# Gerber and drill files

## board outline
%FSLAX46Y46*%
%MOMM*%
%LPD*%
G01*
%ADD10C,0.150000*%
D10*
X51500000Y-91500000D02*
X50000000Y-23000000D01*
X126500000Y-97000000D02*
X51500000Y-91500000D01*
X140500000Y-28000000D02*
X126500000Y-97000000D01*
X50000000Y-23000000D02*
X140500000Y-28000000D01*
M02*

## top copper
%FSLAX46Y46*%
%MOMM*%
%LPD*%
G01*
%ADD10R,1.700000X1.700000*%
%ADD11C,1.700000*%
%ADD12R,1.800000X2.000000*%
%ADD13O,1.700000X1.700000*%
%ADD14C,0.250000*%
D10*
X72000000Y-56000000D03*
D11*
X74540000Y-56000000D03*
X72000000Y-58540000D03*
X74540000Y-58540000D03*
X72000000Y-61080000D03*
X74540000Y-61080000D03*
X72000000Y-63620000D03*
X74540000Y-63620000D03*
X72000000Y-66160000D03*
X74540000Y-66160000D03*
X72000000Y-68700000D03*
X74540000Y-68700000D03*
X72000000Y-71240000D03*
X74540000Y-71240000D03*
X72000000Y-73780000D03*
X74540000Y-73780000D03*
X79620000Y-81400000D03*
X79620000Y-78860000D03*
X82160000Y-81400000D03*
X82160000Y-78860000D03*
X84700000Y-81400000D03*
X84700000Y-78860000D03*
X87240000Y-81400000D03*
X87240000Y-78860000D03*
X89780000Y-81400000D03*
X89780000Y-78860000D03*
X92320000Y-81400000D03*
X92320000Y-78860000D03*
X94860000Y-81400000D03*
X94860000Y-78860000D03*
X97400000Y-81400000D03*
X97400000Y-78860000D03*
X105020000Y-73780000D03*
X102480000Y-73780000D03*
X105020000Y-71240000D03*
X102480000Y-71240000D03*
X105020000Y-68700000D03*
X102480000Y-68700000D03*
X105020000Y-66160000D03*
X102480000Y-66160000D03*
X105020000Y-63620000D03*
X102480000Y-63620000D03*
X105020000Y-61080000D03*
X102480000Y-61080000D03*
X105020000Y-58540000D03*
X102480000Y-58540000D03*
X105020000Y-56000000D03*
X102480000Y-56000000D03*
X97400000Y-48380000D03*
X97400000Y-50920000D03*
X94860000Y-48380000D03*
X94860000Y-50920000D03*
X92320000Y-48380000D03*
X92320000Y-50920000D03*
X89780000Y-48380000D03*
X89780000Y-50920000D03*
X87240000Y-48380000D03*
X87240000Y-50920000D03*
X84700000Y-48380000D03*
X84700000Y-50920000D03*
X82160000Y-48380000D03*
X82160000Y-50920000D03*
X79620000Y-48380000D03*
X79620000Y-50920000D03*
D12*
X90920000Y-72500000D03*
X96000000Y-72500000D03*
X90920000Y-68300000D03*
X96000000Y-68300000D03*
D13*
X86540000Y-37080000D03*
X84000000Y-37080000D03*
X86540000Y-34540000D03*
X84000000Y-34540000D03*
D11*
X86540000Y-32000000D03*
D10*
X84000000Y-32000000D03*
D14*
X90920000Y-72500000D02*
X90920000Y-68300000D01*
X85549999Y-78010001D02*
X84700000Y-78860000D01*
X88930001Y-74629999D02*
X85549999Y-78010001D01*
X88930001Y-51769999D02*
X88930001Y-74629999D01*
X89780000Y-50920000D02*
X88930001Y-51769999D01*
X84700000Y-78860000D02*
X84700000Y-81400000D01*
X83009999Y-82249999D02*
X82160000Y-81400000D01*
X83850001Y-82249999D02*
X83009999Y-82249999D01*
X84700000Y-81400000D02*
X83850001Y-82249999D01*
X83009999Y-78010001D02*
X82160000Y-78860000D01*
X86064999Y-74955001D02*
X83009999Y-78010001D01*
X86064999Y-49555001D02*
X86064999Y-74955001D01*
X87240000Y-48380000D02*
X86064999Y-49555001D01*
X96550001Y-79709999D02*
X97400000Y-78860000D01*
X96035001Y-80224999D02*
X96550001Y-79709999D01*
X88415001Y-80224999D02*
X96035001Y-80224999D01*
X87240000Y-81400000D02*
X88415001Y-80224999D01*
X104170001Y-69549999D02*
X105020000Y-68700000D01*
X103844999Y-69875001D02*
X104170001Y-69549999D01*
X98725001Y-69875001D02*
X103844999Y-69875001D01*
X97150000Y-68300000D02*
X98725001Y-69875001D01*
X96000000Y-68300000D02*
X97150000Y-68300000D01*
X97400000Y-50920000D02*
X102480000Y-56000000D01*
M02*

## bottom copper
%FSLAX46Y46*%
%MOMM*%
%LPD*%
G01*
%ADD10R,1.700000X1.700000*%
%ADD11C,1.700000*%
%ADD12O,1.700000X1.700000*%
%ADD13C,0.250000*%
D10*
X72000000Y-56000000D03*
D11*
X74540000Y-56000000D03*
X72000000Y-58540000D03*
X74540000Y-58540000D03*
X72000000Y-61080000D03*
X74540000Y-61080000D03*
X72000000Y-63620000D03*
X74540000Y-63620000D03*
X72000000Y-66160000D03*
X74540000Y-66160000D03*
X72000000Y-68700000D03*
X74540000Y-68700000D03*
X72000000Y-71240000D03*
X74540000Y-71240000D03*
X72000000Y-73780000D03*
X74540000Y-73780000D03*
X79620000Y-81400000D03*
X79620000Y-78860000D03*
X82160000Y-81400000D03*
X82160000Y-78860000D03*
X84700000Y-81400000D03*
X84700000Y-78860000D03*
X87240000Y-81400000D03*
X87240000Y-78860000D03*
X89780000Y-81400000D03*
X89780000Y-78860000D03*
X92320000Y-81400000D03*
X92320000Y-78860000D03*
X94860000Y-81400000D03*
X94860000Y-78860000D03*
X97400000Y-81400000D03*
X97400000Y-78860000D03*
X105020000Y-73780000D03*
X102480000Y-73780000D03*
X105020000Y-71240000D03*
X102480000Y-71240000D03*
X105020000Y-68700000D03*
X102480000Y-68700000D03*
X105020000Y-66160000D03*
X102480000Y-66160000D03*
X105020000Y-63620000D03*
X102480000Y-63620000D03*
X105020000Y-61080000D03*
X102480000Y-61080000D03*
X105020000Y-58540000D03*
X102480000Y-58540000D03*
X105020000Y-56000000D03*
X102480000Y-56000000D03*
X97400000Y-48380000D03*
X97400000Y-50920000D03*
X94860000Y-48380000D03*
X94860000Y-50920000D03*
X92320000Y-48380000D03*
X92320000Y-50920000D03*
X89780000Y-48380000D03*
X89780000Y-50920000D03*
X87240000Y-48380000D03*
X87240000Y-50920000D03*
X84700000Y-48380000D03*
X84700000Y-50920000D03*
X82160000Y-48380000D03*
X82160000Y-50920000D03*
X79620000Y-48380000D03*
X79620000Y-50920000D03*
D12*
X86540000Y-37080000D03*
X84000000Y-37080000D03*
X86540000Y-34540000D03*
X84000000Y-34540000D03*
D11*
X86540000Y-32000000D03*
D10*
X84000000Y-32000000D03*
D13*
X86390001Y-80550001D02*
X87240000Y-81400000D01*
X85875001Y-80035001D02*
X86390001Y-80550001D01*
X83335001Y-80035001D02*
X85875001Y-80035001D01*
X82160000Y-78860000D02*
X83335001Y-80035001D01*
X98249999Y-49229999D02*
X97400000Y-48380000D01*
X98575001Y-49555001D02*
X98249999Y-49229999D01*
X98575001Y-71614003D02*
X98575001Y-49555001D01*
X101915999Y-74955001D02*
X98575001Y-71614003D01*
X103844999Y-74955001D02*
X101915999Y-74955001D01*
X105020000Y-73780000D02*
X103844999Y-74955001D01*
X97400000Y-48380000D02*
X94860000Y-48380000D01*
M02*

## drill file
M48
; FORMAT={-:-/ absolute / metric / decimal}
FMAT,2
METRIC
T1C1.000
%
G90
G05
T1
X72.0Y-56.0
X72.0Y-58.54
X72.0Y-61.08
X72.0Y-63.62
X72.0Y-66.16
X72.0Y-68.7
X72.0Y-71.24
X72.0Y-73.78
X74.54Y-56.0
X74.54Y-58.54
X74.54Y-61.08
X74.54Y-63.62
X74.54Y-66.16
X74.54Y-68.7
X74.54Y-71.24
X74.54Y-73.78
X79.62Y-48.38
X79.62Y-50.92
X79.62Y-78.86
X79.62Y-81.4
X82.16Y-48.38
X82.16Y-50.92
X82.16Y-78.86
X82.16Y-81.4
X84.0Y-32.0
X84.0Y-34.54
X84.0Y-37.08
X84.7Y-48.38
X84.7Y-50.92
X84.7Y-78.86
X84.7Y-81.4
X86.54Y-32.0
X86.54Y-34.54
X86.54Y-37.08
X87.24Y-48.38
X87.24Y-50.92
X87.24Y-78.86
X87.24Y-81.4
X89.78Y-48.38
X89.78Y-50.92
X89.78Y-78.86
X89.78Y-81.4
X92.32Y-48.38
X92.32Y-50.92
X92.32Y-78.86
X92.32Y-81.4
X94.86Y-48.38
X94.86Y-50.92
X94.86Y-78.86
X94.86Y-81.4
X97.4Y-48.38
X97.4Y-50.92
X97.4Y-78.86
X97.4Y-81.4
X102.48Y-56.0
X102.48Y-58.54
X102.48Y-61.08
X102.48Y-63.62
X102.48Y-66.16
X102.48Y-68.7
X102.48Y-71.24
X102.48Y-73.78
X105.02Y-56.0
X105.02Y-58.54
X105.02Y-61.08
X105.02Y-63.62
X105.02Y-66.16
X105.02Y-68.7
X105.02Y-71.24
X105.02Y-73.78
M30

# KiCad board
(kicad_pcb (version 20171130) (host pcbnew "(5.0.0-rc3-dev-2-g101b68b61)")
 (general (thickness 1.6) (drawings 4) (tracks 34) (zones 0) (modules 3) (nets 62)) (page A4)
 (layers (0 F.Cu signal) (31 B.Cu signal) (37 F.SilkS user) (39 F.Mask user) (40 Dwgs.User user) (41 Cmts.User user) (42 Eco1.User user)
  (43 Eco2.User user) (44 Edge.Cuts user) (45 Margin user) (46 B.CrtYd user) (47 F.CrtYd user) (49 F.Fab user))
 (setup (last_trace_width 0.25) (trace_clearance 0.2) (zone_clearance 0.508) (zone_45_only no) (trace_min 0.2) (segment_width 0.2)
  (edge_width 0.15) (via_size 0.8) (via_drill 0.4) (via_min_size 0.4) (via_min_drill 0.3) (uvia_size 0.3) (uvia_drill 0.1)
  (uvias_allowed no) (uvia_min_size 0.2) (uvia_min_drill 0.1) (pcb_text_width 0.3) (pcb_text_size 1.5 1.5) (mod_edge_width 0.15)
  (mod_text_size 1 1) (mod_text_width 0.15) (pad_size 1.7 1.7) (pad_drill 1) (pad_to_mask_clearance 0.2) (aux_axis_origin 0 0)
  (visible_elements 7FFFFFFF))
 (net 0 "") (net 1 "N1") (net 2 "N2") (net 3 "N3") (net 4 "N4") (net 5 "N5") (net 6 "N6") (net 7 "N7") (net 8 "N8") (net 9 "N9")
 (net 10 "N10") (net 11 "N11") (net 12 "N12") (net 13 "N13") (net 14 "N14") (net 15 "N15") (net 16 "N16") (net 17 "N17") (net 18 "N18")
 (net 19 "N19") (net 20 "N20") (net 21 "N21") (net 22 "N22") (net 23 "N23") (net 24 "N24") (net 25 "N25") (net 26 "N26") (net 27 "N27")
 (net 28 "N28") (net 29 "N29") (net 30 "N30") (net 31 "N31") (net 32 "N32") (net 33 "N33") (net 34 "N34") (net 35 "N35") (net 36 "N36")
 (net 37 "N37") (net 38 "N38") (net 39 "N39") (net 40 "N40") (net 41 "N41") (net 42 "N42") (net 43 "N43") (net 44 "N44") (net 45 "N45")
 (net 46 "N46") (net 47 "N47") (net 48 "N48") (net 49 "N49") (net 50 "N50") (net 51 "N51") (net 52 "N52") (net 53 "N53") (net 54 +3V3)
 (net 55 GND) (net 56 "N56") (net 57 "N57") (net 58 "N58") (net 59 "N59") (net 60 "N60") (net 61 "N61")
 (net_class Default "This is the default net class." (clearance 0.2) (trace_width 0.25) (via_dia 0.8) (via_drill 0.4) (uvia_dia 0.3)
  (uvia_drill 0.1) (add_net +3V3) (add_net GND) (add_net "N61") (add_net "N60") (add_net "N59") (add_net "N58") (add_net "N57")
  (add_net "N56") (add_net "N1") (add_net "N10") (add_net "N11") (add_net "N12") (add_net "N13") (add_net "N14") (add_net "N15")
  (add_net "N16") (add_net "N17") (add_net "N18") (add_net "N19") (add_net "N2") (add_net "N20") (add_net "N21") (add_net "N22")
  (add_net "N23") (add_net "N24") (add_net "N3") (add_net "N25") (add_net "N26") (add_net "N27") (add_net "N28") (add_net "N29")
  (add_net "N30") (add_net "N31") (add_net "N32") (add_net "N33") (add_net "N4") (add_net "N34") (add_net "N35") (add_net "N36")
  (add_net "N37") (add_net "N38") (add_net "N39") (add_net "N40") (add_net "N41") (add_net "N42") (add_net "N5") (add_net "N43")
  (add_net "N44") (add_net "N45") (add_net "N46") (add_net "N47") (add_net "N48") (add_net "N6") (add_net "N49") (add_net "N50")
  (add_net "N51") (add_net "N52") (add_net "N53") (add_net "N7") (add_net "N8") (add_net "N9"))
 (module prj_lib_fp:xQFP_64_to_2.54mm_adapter (layer F.Cu) (at 72 56)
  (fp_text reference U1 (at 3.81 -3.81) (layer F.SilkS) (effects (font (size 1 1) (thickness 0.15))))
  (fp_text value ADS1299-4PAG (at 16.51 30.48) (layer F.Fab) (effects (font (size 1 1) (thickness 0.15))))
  (pad 1 thru_hole rect (at 0 0) (size 1.7 1.7) (drill 1) (layers *.Cu *.Mask) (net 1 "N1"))
  (pad 2 thru_hole circle (at 2.54 0) (size 1.7 1.7) (drill 1) (layers *.Cu *.Mask) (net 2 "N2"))
  (pad 3 thru_hole circle (at 0 2.54) (size 1.7 1.7) (drill 1) (layers *.Cu *.Mask) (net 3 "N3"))
  (pad 4 thru_hole circle (at 2.54 2.54) (size 1.7 1.7) (drill 1) (layers *.Cu *.Mask) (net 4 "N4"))
  (pad 5 thru_hole circle (at 0 5.08) (size 1.7 1.7) (drill 1) (layers *.Cu *.Mask) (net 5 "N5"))
  (pad 6 thru_hole circle (at 2.54 5.08) (size 1.7 1.7) (drill 1) (layers *.Cu *.Mask) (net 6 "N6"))
  (pad 7 thru_hole circle (at 0 7.62) (size 1.7 1.7) (drill 1) (layers *.Cu *.Mask) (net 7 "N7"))
  (pad 8 thru_hole circle (at 2.54 7.62) (size 1.7 1.7) (drill 1) (layers *.Cu *.Mask) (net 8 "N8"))
  (pad 9 thru_hole circle (at 0 10.16) (size 1.7 1.7) (drill 1) (layers *.Cu *.Mask) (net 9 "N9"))
  (pad 10 thru_hole circle (at 2.54 10.16) (size 1.7 1.7) (drill 1) (layers *.Cu *.Mask) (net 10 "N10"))
  (pad 11 thru_hole circle (at 0 12.7) (size 1.7 1.7) (drill 1) (layers *.Cu *.Mask) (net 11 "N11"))
  (pad 12 thru_hole circle (at 2.54 12.7) (size 1.7 1.7) (drill 1) (layers *.Cu *.Mask) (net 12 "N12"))
  (pad 13 thru_hole circle (at 0 15.24) (size 1.7 1.7) (drill 1) (layers *.Cu *.Mask) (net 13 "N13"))
  (pad 14 thru_hole circle (at 2.54 15.24) (size 1.7 1.7) (drill 1) (layers *.Cu *.Mask) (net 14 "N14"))
  (pad 15 thru_hole circle (at 0 17.78) (size 1.7 1.7) (drill 1) (layers *.Cu *.Mask) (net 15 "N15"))
  (pad 16 thru_hole circle (at 2.54 17.78) (size 1.7 1.7) (drill 1) (layers *.Cu *.Mask) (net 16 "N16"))
  (pad 17 thru_hole circle (at 7.62 25.4) (size 1.7 1.7) (drill 1) (layers *.Cu *.Mask) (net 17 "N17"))
  (pad 18 thru_hole circle (at 7.62 22.86) (size 1.7 1.7) (drill 1) (layers *.Cu *.Mask) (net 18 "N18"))
  (pad 19 thru_hole circle (at 10.16 25.4) (size 1.7 1.7) (drill 1) (layers *.Cu *.Mask) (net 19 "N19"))
  (pad 20 thru_hole circle (at 10.16 22.86) (size 1.7 1.7) (drill 1) (layers *.Cu *.Mask) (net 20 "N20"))
  (pad 21 thru_hole circle (at 12.7 25.4) (size 1.7 1.7) (drill 1) (layers *.Cu *.Mask) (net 19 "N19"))
  (pad 22 thru_hole circle (at 12.7 22.86) (size 1.7 1.7) (drill 1) (layers *.Cu *.Mask) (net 19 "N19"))
  (pad 23 thru_hole circle (at 15.24 25.4) (size 1.7 1.7) (drill 1) (layers *.Cu *.Mask) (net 20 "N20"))
  (pad 24 thru_hole circle (at 15.24 22.86) (size 1.7 1.7) (drill 1) (layers *.Cu *.Mask) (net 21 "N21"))
  (pad 25 thru_hole circle (at 17.78 25.4) (size 1.7 1.7) (drill 1) (layers *.Cu *.Mask) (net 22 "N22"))
  (pad 26 thru_hole circle (at 17.78 22.86) (size 1.7 1.7) (drill 1) (layers *.Cu *.Mask) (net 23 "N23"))
  (pad 27 thru_hole circle (at 20.32 25.4) (size 1.7 1.7) (drill 1) (layers *.Cu *.Mask))
  (pad 28 thru_hole circle (at 20.32 22.86) (size 1.7 1.7) (drill 1) (layers *.Cu *.Mask) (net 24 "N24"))
  (pad 29 thru_hole circle (at 22.86 25.4) (size 1.7 1.7) (drill 1) (layers *.Cu *.Mask))
  (pad 30 thru_hole circle (at 22.86 22.86) (size 1.7 1.7) (drill 1) (layers *.Cu *.Mask) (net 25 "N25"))
  (pad 31 thru_hole circle (at 25.4 25.4) (size 1.7 1.7) (drill 1) (layers *.Cu *.Mask) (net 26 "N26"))
  (pad 32 thru_hole circle (at 25.4 22.86) (size 1.7 1.7) (drill 1) (layers *.Cu *.Mask) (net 20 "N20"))
  (pad 33 thru_hole circle (at 33.02 17.78) (size 1.7 1.7) (drill 1) (layers *.Cu *.Mask) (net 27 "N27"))
  (pad 34 thru_hole circle (at 30.48 17.78) (size 1.7 1.7) (drill 1) (layers *.Cu *.Mask) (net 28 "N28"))
  (pad 35 thru_hole circle (at 33.02 15.24) (size 1.7 1.7) (drill 1) (layers *.Cu *.Mask) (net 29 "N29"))
  (pad 36 thru_hole circle (at 30.48 15.24) (size 1.7 1.7) (drill 1) (layers *.Cu *.Mask) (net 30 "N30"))
  (pad 37 thru_hole circle (at 33.02 12.7) (size 1.7 1.7) (drill 1) (layers *.Cu *.Mask) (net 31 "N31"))
  (pad 38 thru_hole circle (at 30.48 12.7) (size 1.7 1.7) (drill 1) (layers *.Cu *.Mask) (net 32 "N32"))
  (pad 39 thru_hole circle (at 33.02 10.16) (size 1.7 1.7) (drill 1) (layers *.Cu *.Mask) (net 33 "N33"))
  (pad 40 thru_hole circle (at 30.48 10.16) (size 1.7 1.7) (drill 1) (layers *.Cu *.Mask) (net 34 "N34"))
  (pad 41 thru_hole circle (at 33.02 7.62) (size 1.7 1.7) (drill 1) (layers *.Cu *.Mask) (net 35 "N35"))
  (pad 42 thru_hole circle (at 30.48 7.62) (size 1.7 1.7) (drill 1) (layers *.Cu *.Mask) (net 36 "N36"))
  (pad 43 thru_hole circle (at 33.02 5.08) (size 1.7 1.7) (drill 1) (layers *.Cu *.Mask) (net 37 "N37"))
  (pad 44 thru_hole circle (at 30.48 5.08) (size 1.7 1.7) (drill 1) (layers *.Cu *.Mask) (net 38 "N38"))
  (pad 45 thru_hole circle (at 33.02 2.54) (size 1.7 1.7) (drill 1) (layers *.Cu *.Mask) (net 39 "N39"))
  (pad 46 thru_hole circle (at 30.48 2.54) (size 1.7 1.7) (drill 1) (layers *.Cu *.Mask) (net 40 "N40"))
  (pad 47 thru_hole circle (at 33.02 0) (size 1.7 1.7) (drill 1) (layers *.Cu *.Mask) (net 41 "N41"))
  (pad 48 thru_hole circle (at 30.48 0) (size 1.7 1.7) (drill 1) (layers *.Cu *.Mask) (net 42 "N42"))
  (pad 49 thru_hole circle (at 25.4 -7.62) (size 1.7 1.7) (drill 1) (layers *.Cu *.Mask) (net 27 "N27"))
  (pad 50 thru_hole circle (at 25.4 -5.08) (size 1.7 1.7) (drill 1) (layers *.Cu *.Mask) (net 42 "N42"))
  (pad 51 thru_hole circle (at 22.86 -7.62) (size 1.7 1.7) (drill 1) (layers *.Cu *.Mask) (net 27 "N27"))
  (pad 52 thru_hole circle (at 22.86 -5.08) (size 1.7 1.7) (drill 1) (layers *.Cu *.Mask) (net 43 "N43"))
  (pad 53 thru_hole circle (at 20.32 -7.62) (size 1.7 1.7) (drill 1) (layers *.Cu *.Mask) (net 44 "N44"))
  (pad 54 thru_hole circle (at 20.32 -5.08) (size 1.7 1.7) (drill 1) (layers *.Cu *.Mask) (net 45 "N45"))
  (pad 55 thru_hole circle (at 17.78 -7.62) (size 1.7 1.7) (drill 1) (layers *.Cu *.Mask) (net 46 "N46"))
  (pad 56 thru_hole circle (at 17.78 -5.08) (size 1.7 1.7) (drill 1) (layers *.Cu *.Mask) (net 19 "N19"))
  (pad 57 thru_hole circle (at 15.24 -7.62) (size 1.7 1.7) (drill 1) (layers *.Cu *.Mask) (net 20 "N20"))
  (pad 58 thru_hole circle (at 15.24 -5.08) (size 1.7 1.7) (drill 1) (layers *.Cu *.Mask) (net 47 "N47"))
  (pad 59 thru_hole circle (at 12.7 -7.62) (size 1.7 1.7) (drill 1) (layers *.Cu *.Mask) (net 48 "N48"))
  (pad 60 thru_hole circle (at 12.7 -5.08) (size 1.7 1.7) (drill 1) (layers *.Cu *.Mask) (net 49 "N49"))
  (pad 61 thru_hole circle (at 10.16 -7.62) (size 1.7 1.7) (drill 1) (layers *.Cu *.Mask) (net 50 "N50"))
  (pad 62 thru_hole circle (at 10.16 -5.08) (size 1.7 1.7) (drill 1) (layers *.Cu *.Mask) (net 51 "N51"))
  (pad 63 thru_hole circle (at 7.62 -7.62) (size 1.7 1.7) (drill 1) (layers *.Cu *.Mask) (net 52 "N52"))
  (pad 64 thru_hole circle (at 7.62 -5.08) (size 1.7 1.7) (drill 1) (layers *.Cu *.Mask) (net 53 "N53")))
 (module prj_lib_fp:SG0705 (layer F.Cu) (at 93.46 70.4)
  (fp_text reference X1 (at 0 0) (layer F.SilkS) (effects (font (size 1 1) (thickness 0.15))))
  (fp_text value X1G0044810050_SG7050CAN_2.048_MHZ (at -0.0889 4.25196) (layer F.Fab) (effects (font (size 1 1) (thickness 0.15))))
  (pad 1 smd rect (at -2.54 2.1) (size 1.8 2) (layers F.Cu F.Paste F.Mask) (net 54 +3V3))
  (pad 2 smd rect (at 2.54 2.1) (size 1.8 2) (layers F.Cu F.Paste F.Mask) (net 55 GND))
  (pad 4 smd rect (at -2.54 -2.1) (size 1.8 2) (layers F.Cu F.Paste F.Mask) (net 54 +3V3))
  (pad 3 smd rect (at 2.54 -2.1) (size 1.8 2) (layers F.Cu F.Paste F.Mask) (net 31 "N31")))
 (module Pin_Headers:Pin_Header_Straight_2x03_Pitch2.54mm (layer F.Cu) (at 84 32)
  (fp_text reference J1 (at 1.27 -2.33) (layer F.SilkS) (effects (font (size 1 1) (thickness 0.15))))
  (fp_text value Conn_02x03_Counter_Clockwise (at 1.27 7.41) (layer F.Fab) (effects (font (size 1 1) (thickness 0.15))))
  (pad 6 thru_hole oval (at 2.54 5.08) (size 1.7 1.7) (drill 1) (layers *.Cu *.Mask) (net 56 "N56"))
  (pad 5 thru_hole oval (at 0 5.08) (size 1.7 1.7) (drill 1) (layers *.Cu *.Mask) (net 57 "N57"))
  (pad 4 thru_hole oval (at 2.54 2.54) (size 1.7 1.7) (drill 1) (layers *.Cu *.Mask) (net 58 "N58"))
  (pad 3 thru_hole oval (at 0 2.54) (size 1.7 1.7) (drill 1) (layers *.Cu *.Mask) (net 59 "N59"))
  (pad 2 thru_hole circle (at 2.54 0) (size 1.7 1.7) (drill 1) (layers *.Cu *.Mask) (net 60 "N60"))
  (pad 1 thru_hole rect (at 0 0) (size 1.7 1.7) (drill 1) (layers *.Cu *.Mask) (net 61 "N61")))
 (gr_line (start 51.5 91.5) (end 50 23) (layer Edge.Cuts) (width 0.15))
 (gr_line (start 126.5 97) (end 51.5 91.5) (layer Edge.Cuts) (width 0.15))
 (gr_line (start 140.5 28) (end 126.5 97) (layer Edge.Cuts) (width 0.15))
 (gr_line (start 50 23) (end 140.5 28) (layer Edge.Cuts) (width 0.15))
 (segment (start 90.92 72.5) (end 90.92 68.3) (width 0.25) (layer F.Cu) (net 54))
 (segment (start 85.549999 78.010001) (end 84.7 78.86) (width 0.25) (layer F.Cu) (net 19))
 (segment (start 88.930001 74.629999) (end 85.549999 78.010001) (width 0.25) (layer F.Cu) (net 19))
 (segment (start 88.930001 51.769999) (end 88.930001 74.629999) (width 0.25) (layer F.Cu) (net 19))
 (segment (start 89.78 50.92) (end 88.930001 51.769999) (width 0.25) (layer F.Cu) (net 19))
 (segment (start 84.7 78.86) (end 84.7 81.4) (width 0.25) (layer F.Cu) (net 19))
 (segment (start 83.009999 82.249999) (end 82.16 81.4) (width 0.25) (layer F.Cu) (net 19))
 (segment (start 83.850001 82.249999) (end 83.009999 82.249999) (width 0.25) (layer F.Cu) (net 19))
 (segment (start 84.7 81.4) (end 83.850001 82.249999) (width 0.25) (layer F.Cu) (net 19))
 (segment (start 83.009999 78.010001) (end 82.16 78.86) (width 0.25) (layer F.Cu) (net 20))
 (segment (start 86.064999 74.955001) (end 83.009999 78.010001) (width 0.25) (layer F.Cu) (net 20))
 (segment (start 86.064999 49.555001) (end 86.064999 74.955001) (width 0.25) (layer F.Cu) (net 20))
 (segment (start 87.24 48.38) (end 86.064999 49.555001) (width 0.25) (layer F.Cu) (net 20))
 (segment (start 86.390001 80.550001) (end 87.24 81.4) (width 0.25) (layer B.Cu) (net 20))
 (segment (start 85.875001 80.035001) (end 86.390001 80.550001) (width 0.25) (layer B.Cu) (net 20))
 (segment (start 83.335001 80.035001) (end 85.875001 80.035001) (width 0.25) (layer B.Cu) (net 20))
 (segment (start 82.16 78.86) (end 83.335001 80.035001) (width 0.25) (layer B.Cu) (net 20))
 (segment (start 96.550001 79.709999) (end 97.4 78.86) (width 0.25) (layer F.Cu) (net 20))
 (segment (start 96.035001 80.224999) (end 96.550001 79.709999) (width 0.25) (layer F.Cu) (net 20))
 (segment (start 88.415001 80.224999) (end 96.035001 80.224999) (width 0.25) (layer F.Cu) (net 20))
 (segment (start 87.24 81.4) (end 88.415001 80.224999) (width 0.25) (layer F.Cu) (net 20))
 (segment (start 98.249999 49.229999) (end 97.4 48.38) (width 0.25) (layer B.Cu) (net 27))
 (segment (start 98.575001 49.555001) (end 98.249999 49.229999) (width 0.25) (layer B.Cu) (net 27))
 (segment (start 98.575001 71.614003) (end 98.575001 49.555001) (width 0.25) (layer B.Cu) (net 27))
 (segment (start 101.915999 74.955001) (end 98.575001 71.614003) (width 0.25) (layer B.Cu) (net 27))
 (segment (start 103.844999 74.955001) (end 101.915999 74.955001) (width 0.25) (layer B.Cu) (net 27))
 (segment (start 105.02 73.78) (end 103.844999 74.955001) (width 0.25) (layer B.Cu) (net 27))
 (segment (start 97.4 48.38) (end 94.86 48.38) (width 0.25) (layer B.Cu) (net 27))
 (segment (start 104.170001 69.549999) (end 105.02 68.7) (width 0.25) (layer F.Cu) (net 31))
 (segment (start 103.844999 69.875001) (end 104.170001 69.549999) (width 0.25) (layer F.Cu) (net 31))
 (segment (start 98.725001 69.875001) (end 103.844999 69.875001) (width 0.25) (layer F.Cu) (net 31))
 (segment (start 97.15 68.3) (end 98.725001 69.875001) (width 0.25) (layer F.Cu) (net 31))
 (segment (start 96 68.3) (end 97.15 68.3) (width 0.25) (layer F.Cu) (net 31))
 (segment (start 97.4 50.92) (end 102.48 56) (width 0.25) (layer F.Cu) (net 42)))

